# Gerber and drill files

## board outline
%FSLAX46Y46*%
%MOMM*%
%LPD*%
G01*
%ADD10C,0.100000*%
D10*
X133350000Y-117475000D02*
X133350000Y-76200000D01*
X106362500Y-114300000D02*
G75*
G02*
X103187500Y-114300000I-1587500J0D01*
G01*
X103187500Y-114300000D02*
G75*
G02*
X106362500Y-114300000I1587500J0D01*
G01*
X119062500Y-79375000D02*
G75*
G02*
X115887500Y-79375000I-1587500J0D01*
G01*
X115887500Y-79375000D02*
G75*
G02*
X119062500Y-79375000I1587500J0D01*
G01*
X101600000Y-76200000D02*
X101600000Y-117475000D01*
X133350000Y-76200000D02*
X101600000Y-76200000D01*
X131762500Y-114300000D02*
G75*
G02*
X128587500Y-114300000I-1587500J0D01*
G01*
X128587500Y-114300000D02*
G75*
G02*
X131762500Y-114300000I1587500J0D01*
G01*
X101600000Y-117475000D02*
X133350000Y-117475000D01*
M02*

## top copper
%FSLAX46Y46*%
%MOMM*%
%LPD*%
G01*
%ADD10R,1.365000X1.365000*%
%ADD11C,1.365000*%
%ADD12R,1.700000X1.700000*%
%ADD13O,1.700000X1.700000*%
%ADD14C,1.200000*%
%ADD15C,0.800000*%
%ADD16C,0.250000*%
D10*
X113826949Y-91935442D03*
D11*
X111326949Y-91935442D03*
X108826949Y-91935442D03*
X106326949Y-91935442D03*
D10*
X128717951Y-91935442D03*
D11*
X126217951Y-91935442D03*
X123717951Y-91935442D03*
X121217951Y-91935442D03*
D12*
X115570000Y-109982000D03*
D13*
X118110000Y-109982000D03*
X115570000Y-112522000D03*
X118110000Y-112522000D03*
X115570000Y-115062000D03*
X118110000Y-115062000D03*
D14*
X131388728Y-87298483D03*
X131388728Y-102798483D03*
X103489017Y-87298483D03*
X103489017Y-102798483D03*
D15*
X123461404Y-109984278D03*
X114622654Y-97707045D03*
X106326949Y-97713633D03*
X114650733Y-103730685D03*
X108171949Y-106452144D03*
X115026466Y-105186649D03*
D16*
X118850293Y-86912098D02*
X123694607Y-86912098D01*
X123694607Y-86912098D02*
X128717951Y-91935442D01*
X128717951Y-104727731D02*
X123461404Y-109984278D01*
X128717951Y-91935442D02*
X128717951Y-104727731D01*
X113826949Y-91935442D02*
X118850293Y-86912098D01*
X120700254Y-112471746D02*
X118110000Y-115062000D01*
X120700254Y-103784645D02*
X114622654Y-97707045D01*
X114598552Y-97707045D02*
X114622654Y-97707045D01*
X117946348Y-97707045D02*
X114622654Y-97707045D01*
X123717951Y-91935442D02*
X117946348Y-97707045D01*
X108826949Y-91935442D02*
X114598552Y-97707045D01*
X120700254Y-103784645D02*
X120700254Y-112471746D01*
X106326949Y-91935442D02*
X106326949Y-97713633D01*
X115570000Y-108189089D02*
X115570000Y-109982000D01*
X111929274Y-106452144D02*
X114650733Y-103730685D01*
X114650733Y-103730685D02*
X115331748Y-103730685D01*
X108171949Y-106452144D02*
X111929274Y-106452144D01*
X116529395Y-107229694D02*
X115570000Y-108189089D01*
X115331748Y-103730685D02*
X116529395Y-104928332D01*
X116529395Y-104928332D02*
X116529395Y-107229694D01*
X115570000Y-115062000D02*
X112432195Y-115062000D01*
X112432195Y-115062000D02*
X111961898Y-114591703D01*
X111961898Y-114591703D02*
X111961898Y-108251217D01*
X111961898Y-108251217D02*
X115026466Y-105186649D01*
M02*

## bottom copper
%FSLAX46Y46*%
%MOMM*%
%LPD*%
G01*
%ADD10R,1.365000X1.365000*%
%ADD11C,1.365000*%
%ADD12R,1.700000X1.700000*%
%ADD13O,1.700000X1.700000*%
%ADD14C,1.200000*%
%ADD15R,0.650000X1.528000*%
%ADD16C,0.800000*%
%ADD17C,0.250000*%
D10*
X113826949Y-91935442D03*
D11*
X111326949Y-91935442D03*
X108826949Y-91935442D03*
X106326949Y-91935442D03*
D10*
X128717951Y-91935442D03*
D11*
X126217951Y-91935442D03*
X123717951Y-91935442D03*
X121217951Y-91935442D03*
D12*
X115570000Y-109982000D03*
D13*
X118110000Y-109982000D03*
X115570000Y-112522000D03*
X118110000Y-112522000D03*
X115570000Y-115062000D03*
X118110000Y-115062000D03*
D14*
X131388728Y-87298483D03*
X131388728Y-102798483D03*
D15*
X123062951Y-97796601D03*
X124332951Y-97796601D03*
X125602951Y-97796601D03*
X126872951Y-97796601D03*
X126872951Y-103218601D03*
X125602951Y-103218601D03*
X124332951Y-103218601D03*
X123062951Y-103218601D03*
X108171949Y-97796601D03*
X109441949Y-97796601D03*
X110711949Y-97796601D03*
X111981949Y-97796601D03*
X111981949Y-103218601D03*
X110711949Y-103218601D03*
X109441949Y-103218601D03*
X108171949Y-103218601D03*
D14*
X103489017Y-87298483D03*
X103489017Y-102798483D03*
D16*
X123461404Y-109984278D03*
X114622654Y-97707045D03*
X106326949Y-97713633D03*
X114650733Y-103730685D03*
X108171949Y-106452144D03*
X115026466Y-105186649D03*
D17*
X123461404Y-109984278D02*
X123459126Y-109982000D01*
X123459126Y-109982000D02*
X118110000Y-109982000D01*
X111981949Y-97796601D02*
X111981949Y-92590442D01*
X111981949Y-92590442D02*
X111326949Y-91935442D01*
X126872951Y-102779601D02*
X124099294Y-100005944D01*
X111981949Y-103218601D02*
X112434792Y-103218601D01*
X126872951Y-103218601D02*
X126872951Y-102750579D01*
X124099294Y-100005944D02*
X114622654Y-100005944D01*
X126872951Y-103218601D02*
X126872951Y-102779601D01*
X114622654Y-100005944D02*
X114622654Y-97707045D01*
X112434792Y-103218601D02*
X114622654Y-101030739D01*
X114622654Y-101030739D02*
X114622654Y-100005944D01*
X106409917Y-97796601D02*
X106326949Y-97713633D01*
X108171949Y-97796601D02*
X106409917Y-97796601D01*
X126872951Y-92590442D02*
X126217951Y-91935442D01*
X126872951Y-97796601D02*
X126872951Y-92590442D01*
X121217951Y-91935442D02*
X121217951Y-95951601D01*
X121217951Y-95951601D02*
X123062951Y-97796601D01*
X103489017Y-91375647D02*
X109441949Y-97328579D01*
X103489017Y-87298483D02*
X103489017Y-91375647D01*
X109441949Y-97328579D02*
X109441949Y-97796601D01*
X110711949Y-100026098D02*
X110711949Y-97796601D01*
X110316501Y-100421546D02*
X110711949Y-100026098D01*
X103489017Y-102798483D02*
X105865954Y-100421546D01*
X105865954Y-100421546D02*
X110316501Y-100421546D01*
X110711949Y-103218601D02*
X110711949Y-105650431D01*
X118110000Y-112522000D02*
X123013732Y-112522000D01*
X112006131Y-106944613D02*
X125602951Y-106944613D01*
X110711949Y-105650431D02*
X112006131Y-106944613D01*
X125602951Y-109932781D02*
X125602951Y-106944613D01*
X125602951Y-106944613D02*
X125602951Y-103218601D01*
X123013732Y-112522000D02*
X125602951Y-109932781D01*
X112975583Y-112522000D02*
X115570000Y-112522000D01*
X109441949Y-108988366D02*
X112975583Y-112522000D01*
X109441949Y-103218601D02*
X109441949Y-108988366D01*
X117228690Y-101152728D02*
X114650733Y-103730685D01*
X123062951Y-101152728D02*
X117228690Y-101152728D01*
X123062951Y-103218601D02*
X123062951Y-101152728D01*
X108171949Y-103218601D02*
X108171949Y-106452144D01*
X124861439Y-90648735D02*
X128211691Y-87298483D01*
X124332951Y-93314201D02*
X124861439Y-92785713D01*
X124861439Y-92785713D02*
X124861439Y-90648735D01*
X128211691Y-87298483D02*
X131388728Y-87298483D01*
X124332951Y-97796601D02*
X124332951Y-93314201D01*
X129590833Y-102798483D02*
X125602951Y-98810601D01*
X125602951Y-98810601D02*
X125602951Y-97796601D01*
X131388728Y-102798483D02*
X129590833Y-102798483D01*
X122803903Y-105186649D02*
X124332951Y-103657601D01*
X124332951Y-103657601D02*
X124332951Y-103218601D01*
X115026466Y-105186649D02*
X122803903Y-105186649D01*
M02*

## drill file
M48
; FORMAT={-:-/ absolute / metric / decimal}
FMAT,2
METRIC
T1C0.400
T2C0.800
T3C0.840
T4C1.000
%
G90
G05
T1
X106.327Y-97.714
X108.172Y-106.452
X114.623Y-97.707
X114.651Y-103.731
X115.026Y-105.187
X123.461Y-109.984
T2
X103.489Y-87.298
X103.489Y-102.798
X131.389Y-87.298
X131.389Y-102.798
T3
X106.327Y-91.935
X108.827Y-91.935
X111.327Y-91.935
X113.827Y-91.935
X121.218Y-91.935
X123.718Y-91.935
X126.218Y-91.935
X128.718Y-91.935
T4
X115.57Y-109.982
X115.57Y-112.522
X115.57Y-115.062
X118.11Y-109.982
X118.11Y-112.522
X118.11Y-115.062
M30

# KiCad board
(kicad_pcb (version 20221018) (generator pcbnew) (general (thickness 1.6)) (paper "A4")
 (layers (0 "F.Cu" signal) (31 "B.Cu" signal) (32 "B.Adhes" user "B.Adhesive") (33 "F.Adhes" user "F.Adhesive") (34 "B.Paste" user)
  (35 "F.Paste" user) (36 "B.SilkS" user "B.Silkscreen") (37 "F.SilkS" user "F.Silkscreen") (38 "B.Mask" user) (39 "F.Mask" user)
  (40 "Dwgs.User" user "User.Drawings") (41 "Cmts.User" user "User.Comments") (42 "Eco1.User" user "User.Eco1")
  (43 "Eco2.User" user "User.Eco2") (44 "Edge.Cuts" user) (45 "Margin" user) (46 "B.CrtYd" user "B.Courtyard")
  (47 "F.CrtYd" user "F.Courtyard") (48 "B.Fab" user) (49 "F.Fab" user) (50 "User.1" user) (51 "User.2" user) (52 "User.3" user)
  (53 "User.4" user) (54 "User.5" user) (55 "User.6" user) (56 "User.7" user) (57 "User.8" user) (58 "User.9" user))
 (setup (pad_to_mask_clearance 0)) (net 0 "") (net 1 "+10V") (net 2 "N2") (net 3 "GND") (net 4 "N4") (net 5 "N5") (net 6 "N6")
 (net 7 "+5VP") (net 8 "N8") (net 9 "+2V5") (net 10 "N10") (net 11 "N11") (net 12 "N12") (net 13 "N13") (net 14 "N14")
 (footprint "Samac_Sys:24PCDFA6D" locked (layer "F.Cu") (at 113.826949 91.935442)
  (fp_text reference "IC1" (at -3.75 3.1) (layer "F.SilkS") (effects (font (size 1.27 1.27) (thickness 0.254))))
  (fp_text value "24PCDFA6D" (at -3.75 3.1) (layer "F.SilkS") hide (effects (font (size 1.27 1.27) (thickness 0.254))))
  (pad "1" thru_hole rect locked (at 0 0) (size 1.365 1.365) (drill 0.84) (layers "*.Cu" "*.Mask") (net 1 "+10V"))
  (pad "2" thru_hole circle locked (at -2.5 0) (size 1.365 1.365) (drill 0.84) (layers "*.Cu" "*.Mask") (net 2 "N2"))
  (pad "3" thru_hole circle locked (at -5 0) (size 1.365 1.365) (drill 0.84) (layers "*.Cu" "*.Mask") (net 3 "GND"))
  (pad "4" thru_hole circle locked (at -7.5 0) (size 1.365 1.365) (drill 0.84) (layers "*.Cu" "*.Mask") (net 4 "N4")))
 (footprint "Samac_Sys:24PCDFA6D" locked (layer "F.Cu") (at 128.717951 91.935442)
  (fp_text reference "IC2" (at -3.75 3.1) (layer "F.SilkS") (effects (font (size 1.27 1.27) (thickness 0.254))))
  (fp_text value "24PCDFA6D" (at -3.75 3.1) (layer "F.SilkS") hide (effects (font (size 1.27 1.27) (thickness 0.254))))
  (pad "1" thru_hole rect locked (at 0 0) (size 1.365 1.365) (drill 0.84) (layers "*.Cu" "*.Mask") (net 1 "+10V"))
  (pad "2" thru_hole circle locked (at -2.5 0) (size 1.365 1.365) (drill 0.84) (layers "*.Cu" "*.Mask") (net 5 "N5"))
  (pad "3" thru_hole circle locked (at -5 0) (size 1.365 1.365) (drill 0.84) (layers "*.Cu" "*.Mask") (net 3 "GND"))
  (pad "4" thru_hole circle locked (at -7.5 0) (size 1.365 1.365) (drill 0.84) (layers "*.Cu" "*.Mask") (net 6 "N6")))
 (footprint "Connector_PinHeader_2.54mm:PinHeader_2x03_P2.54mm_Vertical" (layer "F.Cu") (at 115.57 109.982)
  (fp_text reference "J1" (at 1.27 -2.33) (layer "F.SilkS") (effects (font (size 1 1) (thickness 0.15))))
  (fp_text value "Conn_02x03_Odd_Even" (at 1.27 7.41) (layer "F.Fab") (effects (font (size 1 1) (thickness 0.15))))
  (pad "1" thru_hole rect (at 0 0) (size 1.7 1.7) (drill 1) (layers "*.Cu" "*.Mask") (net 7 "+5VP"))
  (pad "2" thru_hole oval (at 2.54 0) (size 1.7 1.7) (drill 1) (layers "*.Cu" "*.Mask") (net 1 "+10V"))
  (pad "3" thru_hole oval (at 0 2.54) (size 1.7 1.7) (drill 1) (layers "*.Cu" "*.Mask") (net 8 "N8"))
  (pad "4" thru_hole oval (at 2.54 2.54) (size 1.7 1.7) (drill 1) (layers "*.Cu" "*.Mask") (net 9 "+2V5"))
  (pad "5" thru_hole oval (at 0 5.08) (size 1.7 1.7) (drill 1) (layers "*.Cu" "*.Mask") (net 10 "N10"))
  (pad "6" thru_hole oval (at 2.54 5.08) (size 1.7 1.7) (drill 1) (layers "*.Cu" "*.Mask") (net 3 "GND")))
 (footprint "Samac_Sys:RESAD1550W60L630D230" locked (layer "B.Cu") (at 131.388728 87.298483 -90)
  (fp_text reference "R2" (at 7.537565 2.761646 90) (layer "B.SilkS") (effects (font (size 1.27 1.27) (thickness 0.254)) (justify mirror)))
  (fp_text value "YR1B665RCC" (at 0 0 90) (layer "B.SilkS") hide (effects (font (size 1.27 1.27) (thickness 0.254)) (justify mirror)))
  (pad "1" thru_hole circle locked (at 0 0 270) (size 1.2 1.2) (drill 0.8) (layers "*.Cu" "*.Mask") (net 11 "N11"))
  (pad "2" thru_hole circle locked (at 15.5 0 270) (size 1.2 1.2) (drill 0.8) (layers "*.Cu" "*.Mask") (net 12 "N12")))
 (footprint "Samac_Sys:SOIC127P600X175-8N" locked (layer "B.Cu") (at 124.967951 100.507601 -90)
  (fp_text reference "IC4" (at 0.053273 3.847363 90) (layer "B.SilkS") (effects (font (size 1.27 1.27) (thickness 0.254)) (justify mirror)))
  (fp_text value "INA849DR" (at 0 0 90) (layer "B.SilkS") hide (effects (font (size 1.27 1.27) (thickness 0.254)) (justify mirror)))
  (pad "1" smd rect locked (at -2.711 1.905 180) (size 0.65 1.528) (layers "B.Cu" "B.Paste" "B.Mask") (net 6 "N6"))
  (pad "2" smd rect locked (at -2.711 0.635 180) (size 0.65 1.528) (layers "B.Cu" "B.Paste" "B.Mask") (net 11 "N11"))
  (pad "3" smd rect locked (at -2.711 -0.635 180) (size 0.65 1.528) (layers "B.Cu" "B.Paste" "B.Mask") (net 12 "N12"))
  (pad "4" smd rect locked (at -2.711 -1.905 180) (size 0.65 1.528) (layers "B.Cu" "B.Paste" "B.Mask") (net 5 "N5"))
  (pad "5" smd rect locked (at 2.711 -1.905 180) (size 0.65 1.528) (layers "B.Cu" "B.Paste" "B.Mask") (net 3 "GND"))
  (pad "6" smd rect locked (at 2.711 -0.635 180) (size 0.65 1.528) (layers "B.Cu" "B.Paste" "B.Mask") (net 9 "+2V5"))
  (pad "7" smd rect locked (at 2.711 0.635 180) (size 0.65 1.528) (layers "B.Cu" "B.Paste" "B.Mask") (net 10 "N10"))
  (pad "8" smd rect locked (at 2.711 1.905 180) (size 0.65 1.528) (layers "B.Cu" "B.Paste" "B.Mask") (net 7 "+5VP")))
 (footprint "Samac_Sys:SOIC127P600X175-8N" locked (layer "B.Cu") (at 110.076949 100.507601 -90)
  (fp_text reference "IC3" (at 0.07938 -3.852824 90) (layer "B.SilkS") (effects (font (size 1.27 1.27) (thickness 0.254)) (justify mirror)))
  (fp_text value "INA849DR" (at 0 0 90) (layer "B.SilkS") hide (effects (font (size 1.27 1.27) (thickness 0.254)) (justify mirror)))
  (pad "1" smd rect locked (at -2.711 1.905 180) (size 0.65 1.528) (layers "B.Cu" "B.Paste" "B.Mask") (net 4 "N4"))
  (pad "2" smd rect locked (at -2.711 0.635 180) (size 0.65 1.528) (layers "B.Cu" "B.Paste" "B.Mask") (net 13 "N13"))
  (pad "3" smd rect locked (at -2.711 -0.635 180) (size 0.65 1.528) (layers "B.Cu" "B.Paste" "B.Mask") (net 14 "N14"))
  (pad "4" smd rect locked (at -2.711 -1.905 180) (size 0.65 1.528) (layers "B.Cu" "B.Paste" "B.Mask") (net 2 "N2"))
  (pad "5" smd rect locked (at 2.711 -1.905 180) (size 0.65 1.528) (layers "B.Cu" "B.Paste" "B.Mask") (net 3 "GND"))
  (pad "6" smd rect locked (at 2.711 -0.635 180) (size 0.65 1.528) (layers "B.Cu" "B.Paste" "B.Mask") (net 9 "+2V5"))
  (pad "7" smd rect locked (at 2.711 0.635 180) (size 0.65 1.528) (layers "B.Cu" "B.Paste" "B.Mask") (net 8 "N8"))
  (pad "8" smd rect locked (at 2.711 1.905 180) (size 0.65 1.528) (layers "B.Cu" "B.Paste" "B.Mask") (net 7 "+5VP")))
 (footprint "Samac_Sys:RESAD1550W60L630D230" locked (layer "B.Cu") (at 103.489017 87.298483 -90)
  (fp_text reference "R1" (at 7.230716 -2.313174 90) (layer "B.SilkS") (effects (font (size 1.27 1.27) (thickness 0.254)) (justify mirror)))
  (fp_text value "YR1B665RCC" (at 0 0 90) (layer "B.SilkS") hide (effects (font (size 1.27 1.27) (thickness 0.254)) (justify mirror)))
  (pad "1" thru_hole circle locked (at 0 0 270) (size 1.2 1.2) (drill 0.8) (layers "*.Cu" "*.Mask") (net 13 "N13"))
  (pad "2" thru_hole circle locked (at 15.5 0 270) (size 1.2 1.2) (drill 0.8) (layers "*.Cu" "*.Mask") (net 14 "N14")))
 (gr_line (start 133.35 117.475) (end 133.35 76.2) (stroke (width 0.1) (type solid)) (layer "Edge.Cuts"))
 (gr_circle (center 104.775 114.3) (end 106.3625 114.3) (stroke (width 0.1) (type solid)) (fill none) (layer "Edge.Cuts"))
 (gr_circle (center 117.475 79.375) (end 119.0625 79.375) (stroke (width 0.1) (type solid)) (fill none) (layer "Edge.Cuts"))
 (gr_line (start 101.6 76.2) (end 101.6 117.475) (stroke (width 0.1) (type solid)) (layer "Edge.Cuts"))
 (gr_line (start 133.35 76.2) (end 101.6 76.2) (stroke (width 0.1) (type solid)) (layer "Edge.Cuts"))
 (gr_circle (center 130.175 114.3) (end 131.7625 114.3) (stroke (width 0.1) (type solid)) (fill none) (layer "Edge.Cuts"))
 (gr_line (start 101.6 117.475) (end 133.35 117.475) (stroke (width 0.1) (type solid)) (layer "Edge.Cuts"))
 (segment (start 118.850293 86.912098) (end 123.694607 86.912098) (width 0.25) (layer "F.Cu") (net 1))
 (segment (start 123.694607 86.912098) (end 128.717951 91.935442) (width 0.25) (layer "F.Cu") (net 1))
 (segment (start 128.717951 104.727731) (end 123.461404 109.984278) (width 0.25) (layer "F.Cu") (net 1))
 (segment (start 128.717951 91.935442) (end 128.717951 104.727731) (width 0.25) (layer "F.Cu") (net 1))
 (segment (start 113.826949 91.935442) (end 118.850293 86.912098) (width 0.25) (layer "F.Cu") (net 1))
 (via (at 123.461404 109.984278) (size 0.8) (drill 0.4) (layers "F.Cu" "B.Cu") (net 1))
 (segment (start 123.461404 109.984278) (end 123.459126 109.982) (width 0.25) (layer "B.Cu") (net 1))
 (segment (start 123.459126 109.982) (end 118.11 109.982) (width 0.25) (layer "B.Cu") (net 1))
 (segment (start 111.981949 97.796601) (end 111.981949 92.590442) (width 0.25) (layer "B.Cu") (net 2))
 (segment (start 111.981949 92.590442) (end 111.326949 91.935442) (width 0.25) (layer "B.Cu") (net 2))
 (segment (start 120.700254 112.471746) (end 118.11 115.062) (width 0.25) (layer "F.Cu") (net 3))
 (segment (start 120.700254 103.784645) (end 114.622654 97.707045) (width 0.25) (layer "F.Cu") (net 3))
 (segment (start 114.598552 97.707045) (end 114.622654 97.707045) (width 0.25) (layer "F.Cu") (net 3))
 (segment (start 117.946348 97.707045) (end 114.622654 97.707045) (width 0.25) (layer "F.Cu") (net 3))
 (segment (start 123.717951 91.935442) (end 117.946348 97.707045) (width 0.25) (layer "F.Cu") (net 3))
 (segment (start 108.826949 91.935442) (end 114.598552 97.707045) (width 0.25) (layer "F.Cu") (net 3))
 (segment (start 120.700254 103.784645) (end 120.700254 112.471746) (width 0.25) (layer "F.Cu") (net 3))
 (via (at 114.622654 97.707045) (size 0.8) (drill 0.4) (layers "F.Cu" "B.Cu") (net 3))
 (segment (start 126.872951 102.779601) (end 124.099294 100.005944) (width 0.25) (layer "B.Cu") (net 3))
 (segment (start 111.981949 103.218601) (end 112.434792 103.218601) (width 0.25) (layer "B.Cu") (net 3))
 (segment (start 126.872951 103.218601) (end 126.872951 102.750579) (width 0.25) (layer "B.Cu") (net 3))
 (segment (start 124.099294 100.005944) (end 114.622654 100.005944) (width 0.25) (layer "B.Cu") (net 3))
 (segment (start 126.872951 103.218601) (end 126.872951 102.779601) (width 0.25) (layer "B.Cu") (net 3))
 (segment (start 114.622654 100.005944) (end 114.622654 97.707045) (width 0.25) (layer "B.Cu") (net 3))
 (segment (start 112.434792 103.218601) (end 114.622654 101.030739) (width 0.25) (layer "B.Cu") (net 3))
 (segment (start 114.622654 101.030739) (end 114.622654 100.005944) (width 0.25) (layer "B.Cu") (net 3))
 (segment (start 106.326949 91.935442) (end 106.326949 97.713633) (width 0.25) (layer "F.Cu") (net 4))
 (via (at 106.326949 97.713633) (size 0.8) (drill 0.4) (layers "F.Cu" "B.Cu") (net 4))
 (segment (start 106.409917 97.796601) (end 106.326949 97.713633) (width 0.25) (layer "B.Cu") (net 4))
 (segment (start 108.171949 97.796601) (end 106.409917 97.796601) (width 0.25) (layer "B.Cu") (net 4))
 (segment (start 126.872951 92.590442) (end 126.217951 91.935442) (width 0.25) (layer "B.Cu") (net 5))
 (segment (start 126.872951 97.796601) (end 126.872951 92.590442) (width 0.25) (layer "B.Cu") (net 5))
 (segment (start 121.217951 91.935442) (end 121.217951 95.951601) (width 0.25) (layer "B.Cu") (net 6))
 (segment (start 121.217951 95.951601) (end 123.062951 97.796601) (width 0.25) (layer "B.Cu") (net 6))
 (segment (start 103.489017 91.375647) (end 109.441949 97.328579) (width 0.25) (layer "B.Cu") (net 13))
 (segment (start 103.489017 87.298483) (end 103.489017 91.375647) (width 0.25) (layer "B.Cu") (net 13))
 (segment (start 109.441949 97.328579) (end 109.441949 97.796601) (width 0.25) (layer "B.Cu") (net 13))
 (segment (start 110.711949 100.026098) (end 110.711949 97.796601) (width 0.25) (layer "B.Cu") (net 14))
 (segment (start 110.316501 100.421546) (end 110.711949 100.026098) (width 0.25) (layer "B.Cu") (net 14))
 (segment (start 103.489017 102.798483) (end 105.865954 100.421546) (width 0.25) (layer "B.Cu") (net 14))
 (segment (start 105.865954 100.421546) (end 110.316501 100.421546) (width 0.25) (layer "B.Cu") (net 14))
 (segment (start 110.711949 103.218601) (end 110.711949 105.650431) (width 0.25) (layer "B.Cu") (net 9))
 (segment (start 118.11 112.522) (end 123.013732 112.522) (width 0.25) (layer "B.Cu") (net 9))
 (segment (start 112.006131 106.944613) (end 125.602951 106.944613) (width 0.25) (layer "B.Cu") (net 9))
 (segment (start 110.711949 105.650431) (end 112.006131 106.944613) (width 0.25) (layer "B.Cu") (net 9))
 (segment (start 125.602951 109.932781) (end 125.602951 106.944613) (width 0.25) (layer "B.Cu") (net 9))
 (segment (start 125.602951 106.944613) (end 125.602951 103.218601) (width 0.25) (layer "B.Cu") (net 9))
 (segment (start 123.013732 112.522) (end 125.602951 109.932781) (width 0.25) (layer "B.Cu") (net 9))
 (segment (start 112.975583 112.522) (end 115.57 112.522) (width 0.25) (layer "B.Cu") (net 8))
 (segment (start 109.441949 108.988366) (end 112.975583 112.522) (width 0.25) (layer "B.Cu") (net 8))
 (segment (start 109.441949 103.218601) (end 109.441949 108.988366) (width 0.25) (layer "B.Cu") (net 8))
 (segment (start 115.57 108.189089) (end 115.57 109.982) (width 0.25) (layer "F.Cu") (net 7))
 (segment (start 111.929274 106.452144) (end 114.650733 103.730685) (width 0.25) (layer "F.Cu") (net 7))
 (segment (start 114.650733 103.730685) (end 115.331748 103.730685) (width 0.25) (layer "F.Cu") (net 7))
 (segment (start 108.171949 106.452144) (end 111.929274 106.452144) (width 0.25) (layer "F.Cu") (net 7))
 (segment (start 116.529395 107.229694) (end 115.57 108.189089) (width 0.25) (layer "F.Cu") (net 7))
 (segment (start 115.331748 103.730685) (end 116.529395 104.928332) (width 0.25) (layer "F.Cu") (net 7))
 (segment (start 116.529395 104.928332) (end 116.529395 107.229694) (width 0.25) (layer "F.Cu") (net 7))
 (via (at 114.650733 103.730685) (size 0.8) (drill 0.4) (layers "F.Cu" "B.Cu") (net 7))
 (via (at 108.171949 106.452144) (size 0.8) (drill 0.4) (layers "F.Cu" "B.Cu") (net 7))
 (segment (start 117.22869 101.152728) (end 114.650733 103.730685) (width 0.25) (layer "B.Cu") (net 7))
 (segment (start 123.062951 101.152728) (end 117.22869 101.152728) (width 0.25) (layer "B.Cu") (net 7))
 (segment (start 123.062951 103.218601) (end 123.062951 101.152728) (width 0.25) (layer "B.Cu") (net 7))
 (segment (start 108.171949 103.218601) (end 108.171949 106.452144) (width 0.25) (layer "B.Cu") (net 7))
 (segment (start 124.861439 90.648735) (end 128.211691 87.298483) (width 0.25) (layer "B.Cu") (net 11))
 (segment (start 124.332951 93.314201) (end 124.861439 92.785713) (width 0.25) (layer "B.Cu") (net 11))
 (segment (start 124.861439 92.785713) (end 124.861439 90.648735) (width 0.25) (layer "B.Cu") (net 11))
 (segment (start 128.211691 87.298483) (end 131.388728 87.298483) (width 0.25) (layer "B.Cu") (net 11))
 (segment (start 124.332951 97.796601) (end 124.332951 93.314201) (width 0.25) (layer "B.Cu") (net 11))
 (segment (start 129.590833 102.798483) (end 125.602951 98.810601) (width 0.25) (layer "B.Cu") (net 12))
 (segment (start 125.602951 98.810601) (end 125.602951 97.796601) (width 0.25) (layer "B.Cu") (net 12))
 (segment (start 131.388728 102.798483) (end 129.590833 102.798483) (width 0.25) (layer "B.Cu") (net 12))
 (segment (start 115.57 115.062) (end 112.432195 115.062) (width 0.25) (layer "F.Cu") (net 10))
 (segment (start 112.432195 115.062) (end 111.961898 114.591703) (width 0.25) (layer "F.Cu") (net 10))
 (segment (start 111.961898 114.591703) (end 111.961898 108.251217) (width 0.25) (layer "F.Cu") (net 10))
 (segment (start 111.961898 108.251217) (end 115.026466 105.186649) (width 0.25) (layer "F.Cu") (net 10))
 (via (at 115.026466 105.186649) (size 0.8) (drill 0.4) (layers "F.Cu" "B.Cu") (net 10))
 (segment (start 122.803903 105.186649) (end 124.332951 103.657601) (width 0.25) (layer "B.Cu") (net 10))
 (segment (start 124.332951 103.657601) (end 124.332951 103.218601) (width 0.25) (layer "B.Cu") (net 10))
 (segment (start 115.026466 105.186649) (end 122.803903 105.186649) (width 0.25) (layer "B.Cu") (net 10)))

